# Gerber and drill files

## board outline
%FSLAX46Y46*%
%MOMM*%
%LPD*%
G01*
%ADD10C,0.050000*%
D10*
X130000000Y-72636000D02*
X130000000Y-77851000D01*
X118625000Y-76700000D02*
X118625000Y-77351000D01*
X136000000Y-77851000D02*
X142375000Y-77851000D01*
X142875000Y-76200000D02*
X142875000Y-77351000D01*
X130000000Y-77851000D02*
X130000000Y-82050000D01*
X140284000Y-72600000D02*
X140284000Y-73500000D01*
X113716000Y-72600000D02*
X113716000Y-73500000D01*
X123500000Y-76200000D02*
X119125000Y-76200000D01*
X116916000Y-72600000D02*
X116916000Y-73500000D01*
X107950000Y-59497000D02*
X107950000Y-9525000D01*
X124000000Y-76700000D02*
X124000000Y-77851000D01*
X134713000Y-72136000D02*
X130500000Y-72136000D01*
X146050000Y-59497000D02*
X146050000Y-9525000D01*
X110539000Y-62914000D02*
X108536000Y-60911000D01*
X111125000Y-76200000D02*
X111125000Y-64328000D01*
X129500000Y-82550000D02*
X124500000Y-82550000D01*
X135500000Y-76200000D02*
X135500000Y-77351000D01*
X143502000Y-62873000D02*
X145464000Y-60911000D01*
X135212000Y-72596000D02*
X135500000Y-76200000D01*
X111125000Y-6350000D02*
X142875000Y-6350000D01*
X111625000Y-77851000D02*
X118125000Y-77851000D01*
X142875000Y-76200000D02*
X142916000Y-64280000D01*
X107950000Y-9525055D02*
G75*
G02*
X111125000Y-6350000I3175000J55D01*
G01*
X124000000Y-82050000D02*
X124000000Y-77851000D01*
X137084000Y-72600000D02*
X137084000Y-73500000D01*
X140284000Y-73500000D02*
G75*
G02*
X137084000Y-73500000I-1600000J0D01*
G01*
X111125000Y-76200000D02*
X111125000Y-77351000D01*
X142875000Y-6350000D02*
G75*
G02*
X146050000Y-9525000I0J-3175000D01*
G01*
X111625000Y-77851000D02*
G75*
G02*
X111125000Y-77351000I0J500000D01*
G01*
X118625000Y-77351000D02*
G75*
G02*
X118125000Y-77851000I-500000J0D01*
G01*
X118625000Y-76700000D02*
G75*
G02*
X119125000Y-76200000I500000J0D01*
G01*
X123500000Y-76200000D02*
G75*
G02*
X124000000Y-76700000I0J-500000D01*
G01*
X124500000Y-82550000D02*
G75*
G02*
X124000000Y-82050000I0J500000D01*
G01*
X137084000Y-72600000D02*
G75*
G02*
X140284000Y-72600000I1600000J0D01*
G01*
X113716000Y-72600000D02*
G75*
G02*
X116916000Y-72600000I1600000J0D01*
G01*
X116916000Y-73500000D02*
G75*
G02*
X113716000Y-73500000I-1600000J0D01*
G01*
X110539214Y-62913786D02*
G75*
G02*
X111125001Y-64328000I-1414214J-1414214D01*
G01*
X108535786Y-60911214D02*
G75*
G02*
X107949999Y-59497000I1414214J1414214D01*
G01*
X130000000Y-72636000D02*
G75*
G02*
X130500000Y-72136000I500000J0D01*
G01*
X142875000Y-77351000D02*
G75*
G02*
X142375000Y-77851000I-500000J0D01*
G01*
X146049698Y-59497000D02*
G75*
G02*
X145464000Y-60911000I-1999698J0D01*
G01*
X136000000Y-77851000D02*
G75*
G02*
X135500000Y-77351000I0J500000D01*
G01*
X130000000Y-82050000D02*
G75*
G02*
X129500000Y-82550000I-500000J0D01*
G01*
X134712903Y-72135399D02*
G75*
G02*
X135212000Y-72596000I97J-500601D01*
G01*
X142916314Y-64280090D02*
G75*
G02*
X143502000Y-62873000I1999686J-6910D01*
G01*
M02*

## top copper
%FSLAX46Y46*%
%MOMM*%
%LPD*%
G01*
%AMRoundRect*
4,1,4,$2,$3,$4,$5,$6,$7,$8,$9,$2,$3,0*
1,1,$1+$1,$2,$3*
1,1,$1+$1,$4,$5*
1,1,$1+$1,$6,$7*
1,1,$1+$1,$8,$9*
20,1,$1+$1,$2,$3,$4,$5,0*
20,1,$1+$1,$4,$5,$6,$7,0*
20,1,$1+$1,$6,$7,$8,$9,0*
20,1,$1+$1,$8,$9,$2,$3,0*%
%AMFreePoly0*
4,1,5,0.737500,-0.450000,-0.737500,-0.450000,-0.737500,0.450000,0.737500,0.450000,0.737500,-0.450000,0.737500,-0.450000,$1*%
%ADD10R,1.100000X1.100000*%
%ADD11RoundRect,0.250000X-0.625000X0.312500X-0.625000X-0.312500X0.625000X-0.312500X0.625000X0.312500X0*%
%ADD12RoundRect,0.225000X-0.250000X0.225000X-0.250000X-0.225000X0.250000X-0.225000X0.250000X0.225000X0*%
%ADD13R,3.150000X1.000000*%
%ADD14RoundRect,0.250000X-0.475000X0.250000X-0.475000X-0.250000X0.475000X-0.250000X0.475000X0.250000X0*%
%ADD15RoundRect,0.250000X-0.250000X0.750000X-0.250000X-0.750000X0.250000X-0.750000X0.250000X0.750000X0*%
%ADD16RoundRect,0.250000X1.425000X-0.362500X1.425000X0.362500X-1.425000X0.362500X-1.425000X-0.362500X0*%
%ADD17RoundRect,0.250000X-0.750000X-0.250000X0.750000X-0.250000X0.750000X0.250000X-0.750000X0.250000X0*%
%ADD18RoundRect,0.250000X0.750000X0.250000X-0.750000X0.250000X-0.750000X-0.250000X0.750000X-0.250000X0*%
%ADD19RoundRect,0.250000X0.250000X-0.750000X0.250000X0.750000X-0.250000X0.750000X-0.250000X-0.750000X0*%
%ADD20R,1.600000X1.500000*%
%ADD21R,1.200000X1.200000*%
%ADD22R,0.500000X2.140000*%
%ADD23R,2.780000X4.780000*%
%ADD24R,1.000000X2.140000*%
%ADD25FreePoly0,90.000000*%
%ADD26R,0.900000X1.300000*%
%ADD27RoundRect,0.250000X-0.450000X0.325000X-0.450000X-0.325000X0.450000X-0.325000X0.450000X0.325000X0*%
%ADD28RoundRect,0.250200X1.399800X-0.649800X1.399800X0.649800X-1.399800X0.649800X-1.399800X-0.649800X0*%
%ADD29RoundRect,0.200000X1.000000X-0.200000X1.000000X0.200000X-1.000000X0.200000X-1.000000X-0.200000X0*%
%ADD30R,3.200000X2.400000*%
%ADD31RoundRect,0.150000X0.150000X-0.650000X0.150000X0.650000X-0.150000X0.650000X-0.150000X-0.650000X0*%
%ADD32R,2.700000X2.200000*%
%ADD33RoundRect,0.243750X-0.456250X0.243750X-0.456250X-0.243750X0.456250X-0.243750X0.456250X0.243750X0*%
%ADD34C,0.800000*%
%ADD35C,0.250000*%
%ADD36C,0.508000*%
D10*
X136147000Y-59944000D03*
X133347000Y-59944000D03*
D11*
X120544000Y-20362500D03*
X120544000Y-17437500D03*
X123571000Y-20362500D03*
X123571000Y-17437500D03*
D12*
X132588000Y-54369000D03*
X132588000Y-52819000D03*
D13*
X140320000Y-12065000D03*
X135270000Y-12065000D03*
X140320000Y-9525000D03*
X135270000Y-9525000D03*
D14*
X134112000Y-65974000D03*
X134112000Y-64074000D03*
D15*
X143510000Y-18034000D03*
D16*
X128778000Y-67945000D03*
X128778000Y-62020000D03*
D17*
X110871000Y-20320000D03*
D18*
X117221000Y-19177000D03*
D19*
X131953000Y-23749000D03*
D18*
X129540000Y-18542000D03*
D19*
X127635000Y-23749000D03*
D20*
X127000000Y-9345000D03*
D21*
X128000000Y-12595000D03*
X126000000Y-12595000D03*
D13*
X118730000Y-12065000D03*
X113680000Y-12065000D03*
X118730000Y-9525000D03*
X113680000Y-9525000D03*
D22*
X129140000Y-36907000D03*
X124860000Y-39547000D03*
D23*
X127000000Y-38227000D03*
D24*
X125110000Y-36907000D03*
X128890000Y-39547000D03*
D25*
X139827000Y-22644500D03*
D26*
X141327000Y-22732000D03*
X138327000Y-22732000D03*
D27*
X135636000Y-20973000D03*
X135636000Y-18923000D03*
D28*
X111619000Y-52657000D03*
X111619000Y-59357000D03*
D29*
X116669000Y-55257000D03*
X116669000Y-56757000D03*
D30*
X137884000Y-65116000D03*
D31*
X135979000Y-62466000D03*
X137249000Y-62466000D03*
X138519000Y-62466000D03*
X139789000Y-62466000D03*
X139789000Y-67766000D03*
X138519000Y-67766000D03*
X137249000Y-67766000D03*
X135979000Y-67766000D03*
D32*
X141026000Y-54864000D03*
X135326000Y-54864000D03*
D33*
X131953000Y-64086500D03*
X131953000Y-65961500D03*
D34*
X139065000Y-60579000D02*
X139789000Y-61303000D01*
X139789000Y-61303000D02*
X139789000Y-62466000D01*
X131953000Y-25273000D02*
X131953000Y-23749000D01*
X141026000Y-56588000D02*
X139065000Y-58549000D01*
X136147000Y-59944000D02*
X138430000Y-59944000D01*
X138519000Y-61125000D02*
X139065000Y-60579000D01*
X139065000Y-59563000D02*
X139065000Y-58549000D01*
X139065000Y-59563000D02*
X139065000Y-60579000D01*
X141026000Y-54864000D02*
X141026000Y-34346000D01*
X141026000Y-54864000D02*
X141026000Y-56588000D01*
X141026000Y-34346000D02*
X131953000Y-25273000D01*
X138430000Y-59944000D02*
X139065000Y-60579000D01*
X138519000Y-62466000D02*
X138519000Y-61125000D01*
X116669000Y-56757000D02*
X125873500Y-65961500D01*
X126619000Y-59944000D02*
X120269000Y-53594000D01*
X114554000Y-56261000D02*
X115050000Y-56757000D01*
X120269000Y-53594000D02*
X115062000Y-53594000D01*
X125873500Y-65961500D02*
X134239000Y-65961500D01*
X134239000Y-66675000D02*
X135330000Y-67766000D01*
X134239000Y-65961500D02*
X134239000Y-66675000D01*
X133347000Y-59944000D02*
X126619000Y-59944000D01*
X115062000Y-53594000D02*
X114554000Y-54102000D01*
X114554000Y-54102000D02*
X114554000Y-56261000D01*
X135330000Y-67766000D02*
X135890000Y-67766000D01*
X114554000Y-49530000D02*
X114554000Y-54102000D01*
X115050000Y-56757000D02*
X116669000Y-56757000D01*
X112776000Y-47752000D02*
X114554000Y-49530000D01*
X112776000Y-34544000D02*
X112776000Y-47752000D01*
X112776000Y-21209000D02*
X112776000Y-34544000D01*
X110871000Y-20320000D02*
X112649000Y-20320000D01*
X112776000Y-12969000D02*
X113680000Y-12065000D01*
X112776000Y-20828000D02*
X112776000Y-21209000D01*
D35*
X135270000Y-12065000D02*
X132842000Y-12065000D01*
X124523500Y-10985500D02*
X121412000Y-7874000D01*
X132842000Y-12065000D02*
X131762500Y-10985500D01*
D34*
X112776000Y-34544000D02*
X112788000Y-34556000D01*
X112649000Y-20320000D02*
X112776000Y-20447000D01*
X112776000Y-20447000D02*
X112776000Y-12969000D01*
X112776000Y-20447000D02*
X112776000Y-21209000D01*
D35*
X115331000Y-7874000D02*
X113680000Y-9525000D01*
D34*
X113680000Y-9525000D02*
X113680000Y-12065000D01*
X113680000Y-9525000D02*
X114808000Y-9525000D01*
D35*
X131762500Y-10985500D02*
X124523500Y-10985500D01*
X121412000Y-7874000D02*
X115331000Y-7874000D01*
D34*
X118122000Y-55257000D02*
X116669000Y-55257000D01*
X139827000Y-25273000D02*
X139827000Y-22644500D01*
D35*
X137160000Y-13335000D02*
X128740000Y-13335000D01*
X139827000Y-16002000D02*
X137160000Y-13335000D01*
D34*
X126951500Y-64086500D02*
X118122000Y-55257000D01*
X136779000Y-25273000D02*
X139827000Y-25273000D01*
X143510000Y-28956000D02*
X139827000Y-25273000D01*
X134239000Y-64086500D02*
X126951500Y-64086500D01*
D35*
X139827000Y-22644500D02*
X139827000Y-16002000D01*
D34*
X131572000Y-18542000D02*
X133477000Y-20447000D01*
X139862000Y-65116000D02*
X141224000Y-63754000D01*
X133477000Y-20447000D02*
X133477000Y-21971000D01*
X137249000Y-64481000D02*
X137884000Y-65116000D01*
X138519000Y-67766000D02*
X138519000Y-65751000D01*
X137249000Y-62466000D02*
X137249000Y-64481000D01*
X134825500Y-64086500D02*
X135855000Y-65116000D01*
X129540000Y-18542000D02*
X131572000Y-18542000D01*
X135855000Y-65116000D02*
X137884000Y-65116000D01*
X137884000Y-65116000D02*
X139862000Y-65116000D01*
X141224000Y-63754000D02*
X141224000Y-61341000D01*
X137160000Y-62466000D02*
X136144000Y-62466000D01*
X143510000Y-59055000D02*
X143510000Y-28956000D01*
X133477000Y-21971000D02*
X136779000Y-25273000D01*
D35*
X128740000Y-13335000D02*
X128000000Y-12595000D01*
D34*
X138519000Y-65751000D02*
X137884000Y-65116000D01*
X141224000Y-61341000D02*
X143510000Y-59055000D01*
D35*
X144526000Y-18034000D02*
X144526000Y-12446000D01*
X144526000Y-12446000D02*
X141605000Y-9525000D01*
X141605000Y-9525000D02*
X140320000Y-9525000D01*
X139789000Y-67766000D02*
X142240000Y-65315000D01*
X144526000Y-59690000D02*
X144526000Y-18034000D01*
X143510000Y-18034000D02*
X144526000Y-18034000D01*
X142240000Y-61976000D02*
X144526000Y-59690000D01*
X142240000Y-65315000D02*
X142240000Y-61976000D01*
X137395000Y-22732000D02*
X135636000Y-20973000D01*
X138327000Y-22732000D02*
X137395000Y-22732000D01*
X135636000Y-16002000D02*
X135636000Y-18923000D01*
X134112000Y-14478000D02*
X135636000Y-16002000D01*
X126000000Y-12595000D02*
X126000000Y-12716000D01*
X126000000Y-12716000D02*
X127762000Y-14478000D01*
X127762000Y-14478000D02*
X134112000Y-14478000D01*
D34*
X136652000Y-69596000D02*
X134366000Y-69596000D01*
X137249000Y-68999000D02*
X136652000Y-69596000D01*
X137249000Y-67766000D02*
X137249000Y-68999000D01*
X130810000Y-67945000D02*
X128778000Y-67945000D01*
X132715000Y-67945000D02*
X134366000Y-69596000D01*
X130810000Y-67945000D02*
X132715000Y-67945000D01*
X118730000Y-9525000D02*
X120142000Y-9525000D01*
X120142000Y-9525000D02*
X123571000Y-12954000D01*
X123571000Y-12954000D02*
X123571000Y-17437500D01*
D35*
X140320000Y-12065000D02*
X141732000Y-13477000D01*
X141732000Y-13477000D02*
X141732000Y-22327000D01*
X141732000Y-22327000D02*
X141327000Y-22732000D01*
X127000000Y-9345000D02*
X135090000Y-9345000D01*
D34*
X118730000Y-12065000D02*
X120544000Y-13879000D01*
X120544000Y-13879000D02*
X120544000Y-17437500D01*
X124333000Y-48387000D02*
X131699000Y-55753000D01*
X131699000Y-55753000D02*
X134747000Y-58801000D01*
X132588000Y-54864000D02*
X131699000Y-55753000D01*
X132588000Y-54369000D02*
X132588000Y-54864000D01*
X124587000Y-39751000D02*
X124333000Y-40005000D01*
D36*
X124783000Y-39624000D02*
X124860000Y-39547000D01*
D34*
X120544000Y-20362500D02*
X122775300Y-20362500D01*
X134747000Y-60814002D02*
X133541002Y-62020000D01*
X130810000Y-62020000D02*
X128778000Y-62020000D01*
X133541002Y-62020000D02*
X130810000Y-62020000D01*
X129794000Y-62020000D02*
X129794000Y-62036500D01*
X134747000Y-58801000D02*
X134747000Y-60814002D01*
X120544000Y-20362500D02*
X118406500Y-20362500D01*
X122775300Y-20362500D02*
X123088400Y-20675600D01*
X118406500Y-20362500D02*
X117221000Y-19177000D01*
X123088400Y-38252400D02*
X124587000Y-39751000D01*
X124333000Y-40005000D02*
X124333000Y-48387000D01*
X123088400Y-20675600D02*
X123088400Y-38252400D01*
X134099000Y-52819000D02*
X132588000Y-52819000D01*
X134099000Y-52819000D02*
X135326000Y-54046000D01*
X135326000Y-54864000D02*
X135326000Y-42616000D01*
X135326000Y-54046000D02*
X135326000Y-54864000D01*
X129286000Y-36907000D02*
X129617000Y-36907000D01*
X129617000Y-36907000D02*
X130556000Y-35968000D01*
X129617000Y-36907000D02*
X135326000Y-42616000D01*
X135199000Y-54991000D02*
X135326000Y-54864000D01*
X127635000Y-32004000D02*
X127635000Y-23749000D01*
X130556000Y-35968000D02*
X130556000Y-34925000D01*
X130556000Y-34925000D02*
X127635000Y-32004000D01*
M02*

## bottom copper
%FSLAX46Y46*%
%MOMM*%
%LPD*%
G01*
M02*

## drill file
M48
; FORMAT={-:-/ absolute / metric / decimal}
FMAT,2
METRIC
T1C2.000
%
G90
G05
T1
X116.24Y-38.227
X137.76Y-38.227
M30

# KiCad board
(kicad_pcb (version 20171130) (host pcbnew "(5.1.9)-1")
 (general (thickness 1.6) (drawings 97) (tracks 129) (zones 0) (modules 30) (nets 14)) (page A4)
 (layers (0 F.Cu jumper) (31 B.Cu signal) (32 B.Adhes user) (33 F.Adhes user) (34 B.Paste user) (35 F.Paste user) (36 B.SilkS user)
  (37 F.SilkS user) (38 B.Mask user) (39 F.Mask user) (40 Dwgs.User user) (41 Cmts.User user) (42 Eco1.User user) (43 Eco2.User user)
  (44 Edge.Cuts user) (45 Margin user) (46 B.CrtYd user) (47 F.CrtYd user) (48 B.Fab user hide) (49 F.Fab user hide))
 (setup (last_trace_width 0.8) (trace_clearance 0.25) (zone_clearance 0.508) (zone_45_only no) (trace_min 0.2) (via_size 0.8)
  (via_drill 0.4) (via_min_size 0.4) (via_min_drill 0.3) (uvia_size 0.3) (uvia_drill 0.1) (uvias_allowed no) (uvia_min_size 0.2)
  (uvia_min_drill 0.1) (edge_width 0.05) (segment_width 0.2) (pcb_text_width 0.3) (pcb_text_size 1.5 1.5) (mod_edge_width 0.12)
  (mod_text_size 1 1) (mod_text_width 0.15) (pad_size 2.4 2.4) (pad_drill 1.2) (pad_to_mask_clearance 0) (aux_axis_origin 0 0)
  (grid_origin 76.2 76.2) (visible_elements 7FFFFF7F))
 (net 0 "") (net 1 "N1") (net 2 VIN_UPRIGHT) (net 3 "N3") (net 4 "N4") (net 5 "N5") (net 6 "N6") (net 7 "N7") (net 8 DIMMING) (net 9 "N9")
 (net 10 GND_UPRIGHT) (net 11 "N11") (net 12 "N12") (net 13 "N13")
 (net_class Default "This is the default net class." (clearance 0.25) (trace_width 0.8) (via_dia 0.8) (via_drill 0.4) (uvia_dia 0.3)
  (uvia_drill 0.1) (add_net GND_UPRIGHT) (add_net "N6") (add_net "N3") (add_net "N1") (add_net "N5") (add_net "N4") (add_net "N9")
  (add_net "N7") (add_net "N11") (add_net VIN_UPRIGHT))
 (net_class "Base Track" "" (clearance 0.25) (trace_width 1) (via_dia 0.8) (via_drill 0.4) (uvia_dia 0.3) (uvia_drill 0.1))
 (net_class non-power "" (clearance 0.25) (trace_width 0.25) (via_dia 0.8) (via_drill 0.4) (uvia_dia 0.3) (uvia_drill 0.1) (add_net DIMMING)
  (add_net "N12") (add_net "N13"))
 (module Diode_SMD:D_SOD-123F (layer F.Cu) (at 134.747 59.944)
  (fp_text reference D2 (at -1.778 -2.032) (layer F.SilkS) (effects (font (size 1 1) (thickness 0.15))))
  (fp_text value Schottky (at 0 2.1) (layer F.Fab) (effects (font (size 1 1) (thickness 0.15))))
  (pad 2 smd rect (at 1.4 0) (size 1.1 1.1) (layers F.Cu F.Paste F.Mask) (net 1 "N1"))
  (pad 1 smd rect (at -1.4 0) (size 1.1 1.1) (layers F.Cu F.Paste F.Mask) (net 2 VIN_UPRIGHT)))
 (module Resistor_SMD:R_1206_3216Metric (layer F.Cu) (at 120.544 18.9 270)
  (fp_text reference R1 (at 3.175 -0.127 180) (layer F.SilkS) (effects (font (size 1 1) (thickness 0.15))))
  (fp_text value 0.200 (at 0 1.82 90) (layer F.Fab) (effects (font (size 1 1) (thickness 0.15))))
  (pad 2 smd roundrect (at 1.4625 0 270) (size 1.125 1.75) (layers F.Cu F.Paste F.Mask) (roundrect_rratio 0.222222) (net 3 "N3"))
  (pad 1 smd roundrect (at -1.4625 0 270) (size 1.125 1.75) (layers F.Cu F.Paste F.Mask) (roundrect_rratio 0.222222) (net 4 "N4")))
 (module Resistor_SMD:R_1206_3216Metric (layer F.Cu) (at 123.571 18.9 270)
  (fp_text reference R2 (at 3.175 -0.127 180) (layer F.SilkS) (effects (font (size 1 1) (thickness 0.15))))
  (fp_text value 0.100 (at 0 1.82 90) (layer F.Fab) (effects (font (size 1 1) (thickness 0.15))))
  (pad 2 smd roundrect (at 1.4625 0 270) (size 1.125 1.75) (layers F.Cu F.Paste F.Mask) (roundrect_rratio 0.222222) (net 3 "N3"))
  (pad 1 smd roundrect (at -1.4625 0 270) (size 1.125 1.75) (layers F.Cu F.Paste F.Mask) (roundrect_rratio 0.222222) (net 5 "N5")))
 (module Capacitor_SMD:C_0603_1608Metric (layer F.Cu) (at 132.588 53.594 270)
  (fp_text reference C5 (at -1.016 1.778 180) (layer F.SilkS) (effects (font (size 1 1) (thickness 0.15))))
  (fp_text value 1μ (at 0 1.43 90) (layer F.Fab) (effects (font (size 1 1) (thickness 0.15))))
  (pad 2 smd roundrect (at 0.775 0 270) (size 0.9 0.95) (layers F.Cu F.Paste F.Mask) (roundrect_rratio 0.25) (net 3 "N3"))
  (pad 1 smd roundrect (at -0.775 0 270) (size 0.9 0.95) (layers F.Cu F.Paste F.Mask) (roundrect_rratio 0.25) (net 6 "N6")))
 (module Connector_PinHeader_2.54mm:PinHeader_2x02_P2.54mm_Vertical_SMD (layer F.Cu) (at 137.795 10.795)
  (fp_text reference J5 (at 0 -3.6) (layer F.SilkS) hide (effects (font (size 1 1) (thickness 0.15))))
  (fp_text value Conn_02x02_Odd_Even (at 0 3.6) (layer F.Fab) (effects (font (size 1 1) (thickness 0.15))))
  (pad 4 smd rect (at 2.525 1.27) (size 3.15 1) (layers F.Cu F.Paste F.Mask) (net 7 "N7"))
  (pad 3 smd rect (at -2.525 1.27) (size 3.15 1) (layers F.Cu F.Paste F.Mask) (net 2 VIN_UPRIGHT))
  (pad 1 smd rect (at 2.525 -1.27) (size 3.15 1) (layers F.Cu F.Paste F.Mask) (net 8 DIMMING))
  (pad 2 smd rect (at -2.525 -1.27) (size 3.15 1) (layers F.Cu F.Paste F.Mask) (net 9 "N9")))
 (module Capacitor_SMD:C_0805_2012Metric (layer F.Cu) (at 134.112 65.024 270)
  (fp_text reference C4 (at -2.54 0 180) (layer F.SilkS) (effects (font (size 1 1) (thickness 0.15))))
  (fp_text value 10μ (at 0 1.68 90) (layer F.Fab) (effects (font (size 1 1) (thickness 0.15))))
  (pad 2 smd roundrect (at 0.95 0 270) (size 1 1.45) (layers F.Cu F.Paste F.Mask) (roundrect_rratio 0.25) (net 2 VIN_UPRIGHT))
  (pad 1 smd roundrect (at -0.95 0 270) (size 1 1.45) (layers F.Cu F.Paste F.Mask) (roundrect_rratio 0.25) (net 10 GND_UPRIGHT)))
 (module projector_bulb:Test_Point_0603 (layer F.Cu) (at 143.51 18.034 270)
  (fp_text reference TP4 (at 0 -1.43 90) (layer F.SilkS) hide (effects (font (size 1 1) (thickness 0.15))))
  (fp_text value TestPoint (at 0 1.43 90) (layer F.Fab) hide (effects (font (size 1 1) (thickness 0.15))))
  (pad 1 smd roundrect (at 0 0 270) (size 2 1) (layers F.Cu F.Paste F.Mask) (roundrect_rratio 0.25) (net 8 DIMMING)))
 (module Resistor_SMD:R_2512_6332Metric (layer F.Cu) (at 128.778 64.9825 90)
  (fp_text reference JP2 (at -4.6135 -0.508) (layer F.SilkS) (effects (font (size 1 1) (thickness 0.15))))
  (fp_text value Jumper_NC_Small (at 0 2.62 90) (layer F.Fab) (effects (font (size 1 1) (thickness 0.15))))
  (pad 1 smd roundrect (at -2.9625 0 90) (size 1.225 3.35) (layers F.Cu F.Paste F.Mask) (roundrect_rratio 0.204082) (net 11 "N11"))
  (pad 2 smd roundrect (at 2.9625 0 90) (size 1.225 3.35) (layers F.Cu F.Paste F.Mask) (roundrect_rratio 0.204082) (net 3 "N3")))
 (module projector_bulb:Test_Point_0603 (layer F.Cu) (at 110.871 20.32)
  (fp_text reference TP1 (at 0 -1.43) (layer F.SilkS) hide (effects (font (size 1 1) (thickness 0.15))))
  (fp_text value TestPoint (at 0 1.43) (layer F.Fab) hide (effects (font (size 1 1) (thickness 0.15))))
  (pad 1 smd roundrect (at 0 0) (size 2 1) (layers F.Cu F.Paste F.Mask) (roundrect_rratio 0.25) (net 2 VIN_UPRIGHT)))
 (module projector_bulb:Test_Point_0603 (layer F.Cu) (at 117.221 19.177 180)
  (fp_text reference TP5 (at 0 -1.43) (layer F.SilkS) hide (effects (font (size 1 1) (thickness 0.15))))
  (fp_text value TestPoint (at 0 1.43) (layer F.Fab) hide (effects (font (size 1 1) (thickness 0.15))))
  (pad 1 smd roundrect (at 0 0 180) (size 2 1) (layers F.Cu F.Paste F.Mask) (roundrect_rratio 0.25) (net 3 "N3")))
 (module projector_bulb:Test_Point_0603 (layer F.Cu) (at 131.953 23.749 90)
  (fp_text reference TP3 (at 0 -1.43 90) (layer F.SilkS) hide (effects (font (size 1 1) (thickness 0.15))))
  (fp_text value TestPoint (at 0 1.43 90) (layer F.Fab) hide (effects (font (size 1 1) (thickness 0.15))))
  (pad 1 smd roundrect (at 0 0 90) (size 2 1) (layers F.Cu F.Paste F.Mask) (roundrect_rratio 0.25) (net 1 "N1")))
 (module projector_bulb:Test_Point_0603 (layer F.Cu) (at 129.54 18.542 180)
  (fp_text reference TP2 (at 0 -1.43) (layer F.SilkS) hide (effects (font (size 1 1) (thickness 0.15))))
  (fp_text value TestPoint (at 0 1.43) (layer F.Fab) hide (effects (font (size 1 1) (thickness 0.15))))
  (pad 1 smd roundrect (at 0 0 180) (size 2 1) (layers F.Cu F.Paste F.Mask) (roundrect_rratio 0.25) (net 10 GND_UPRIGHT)))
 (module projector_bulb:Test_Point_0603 (layer F.Cu) (at 127.635 23.749 90)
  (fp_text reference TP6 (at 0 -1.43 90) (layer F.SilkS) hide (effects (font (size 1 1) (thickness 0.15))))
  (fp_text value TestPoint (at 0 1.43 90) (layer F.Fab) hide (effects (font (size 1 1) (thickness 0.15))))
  (pad 1 smd roundrect (at 0 0 90) (size 2 1) (layers F.Cu F.Paste F.Mask) (roundrect_rratio 0.25) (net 6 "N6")))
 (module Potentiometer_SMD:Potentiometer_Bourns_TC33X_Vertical (layer F.Cu) (at 127 10.795 90)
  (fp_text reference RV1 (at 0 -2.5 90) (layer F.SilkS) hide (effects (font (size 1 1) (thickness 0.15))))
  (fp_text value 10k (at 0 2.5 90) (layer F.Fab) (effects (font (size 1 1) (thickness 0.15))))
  (pad 2 smd rect (at 1.45 0 90) (size 1.5 1.6) (layers F.Cu F.Paste F.Mask) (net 9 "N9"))
  (pad 3 smd rect (at -1.8 1 90) (size 1.2 1.2) (layers F.Cu F.Paste F.Mask) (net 10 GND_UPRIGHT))
  (pad 1 smd rect (at -1.8 -1 90) (size 1.2 1.2) (layers F.Cu F.Paste F.Mask) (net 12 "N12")))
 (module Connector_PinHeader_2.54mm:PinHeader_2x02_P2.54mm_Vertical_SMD (layer F.Cu) (at 116.205 10.795)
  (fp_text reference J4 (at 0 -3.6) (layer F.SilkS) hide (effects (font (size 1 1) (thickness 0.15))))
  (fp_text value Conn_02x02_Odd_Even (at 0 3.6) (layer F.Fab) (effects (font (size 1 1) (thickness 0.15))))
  (pad 4 smd rect (at 2.525 1.27) (size 3.15 1) (layers F.Cu F.Paste F.Mask) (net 4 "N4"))
  (pad 3 smd rect (at -2.525 1.27) (size 3.15 1) (layers F.Cu F.Paste F.Mask) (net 2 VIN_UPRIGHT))
  (pad 2 smd rect (at 2.525 -1.27) (size 3.15 1) (layers F.Cu F.Paste F.Mask) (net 5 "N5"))
  (pad 1 smd rect (at -2.525 -1.27) (size 3.15 1) (layers F.Cu F.Paste F.Mask) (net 2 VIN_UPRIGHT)))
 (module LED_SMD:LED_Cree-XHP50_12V (layer F.Cu) (at 127 38.227 180)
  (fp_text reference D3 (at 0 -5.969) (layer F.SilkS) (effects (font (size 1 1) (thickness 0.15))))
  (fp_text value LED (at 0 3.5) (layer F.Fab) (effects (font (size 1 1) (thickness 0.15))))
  (pad 1 smd rect (at -2.14 1.32 180) (size 0.5 2.14) (layers F.Cu F.Paste F.Mask) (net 6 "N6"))
  (pad 2 smd rect (at 2.14 -1.32 180) (size 0.5 2.14) (layers F.Cu F.Paste F.Mask) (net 3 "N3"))
  (pad 3 smd rect (at 0 0 180) (size 2.78 4.78) (layers F.Cu F.Mask))
  (pad 3 smd rect (at 1.89 1.32 180) (size 1 2.14) (layers F.Cu F.Mask))
  (pad 3 smd rect (at -1.89 -1.32 180) (size 1 2.14) (layers F.Cu F.Mask))
  (pad "" smd rect (at -2.14 -1.32 180) (size 0.5 2.14) (layers F.Paste))
  (pad "" smd rect (at 2.14 1.32 180) (size 0.5 2.14) (layers F.Paste))
  (pad "" smd rect (at -0.61 -1.575 180) (size 0.97 0.8) (layers F.Paste))
  (pad "" smd rect (at 0.61 -1.575 180) (size 0.97 0.8) (layers F.Paste))
  (pad "" smd rect (at -0.61 -0.525 180) (size 0.97 0.8) (layers F.Paste))
  (pad "" smd rect (at 0.61 -0.525 180) (size 0.97 0.8) (layers F.Paste))
  (pad "" smd rect (at -0.61 0.525 180) (size 0.97 0.8) (layers F.Paste))
  (pad "" smd rect (at 0.61 0.525 180) (size 0.97 0.8) (layers F.Paste))
  (pad "" smd rect (at -0.61 1.575 180) (size 0.97 0.8) (layers F.Paste))
  (pad "" smd rect (at 0.61 1.575 180) (size 0.97 0.8) (layers F.Paste)))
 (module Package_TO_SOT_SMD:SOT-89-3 (layer F.Cu) (at 139.827 21.082 90)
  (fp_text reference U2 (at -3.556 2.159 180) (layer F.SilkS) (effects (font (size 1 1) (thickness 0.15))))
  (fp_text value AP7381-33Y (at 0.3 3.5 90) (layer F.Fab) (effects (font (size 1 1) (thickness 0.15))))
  (pad 2 smd custom (at -1.5625 0 90) (size 1.475 0.9) (layers F.Cu F.Paste F.Mask) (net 10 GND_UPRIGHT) (zone_connect 2)
   (options (clearance outline) (anchor rect)) (primitives))
  (pad 3 smd rect (at -1.65 1.5 90) (size 1.3 0.9) (layers F.Cu F.Paste F.Mask) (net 7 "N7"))
  (pad 1 smd rect (at -1.65 -1.5 90) (size 1.3 0.9) (layers F.Cu F.Paste F.Mask) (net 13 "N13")))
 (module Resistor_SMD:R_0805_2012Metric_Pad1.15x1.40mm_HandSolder (layer F.Cu) (at 135.636 19.948 270)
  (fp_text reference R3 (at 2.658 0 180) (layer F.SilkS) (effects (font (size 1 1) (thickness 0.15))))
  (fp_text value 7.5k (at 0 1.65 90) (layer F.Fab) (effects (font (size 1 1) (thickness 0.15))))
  (pad 2 smd roundrect (at 1.025 0 270) (size 1.15 1.4) (layers F.Cu F.Paste F.Mask) (roundrect_rratio 0.217391) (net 13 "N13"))
  (pad 1 smd roundrect (at -1.025 0 270) (size 1.15 1.4) (layers F.Cu F.Paste F.Mask) (roundrect_rratio 0.217391) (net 12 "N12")))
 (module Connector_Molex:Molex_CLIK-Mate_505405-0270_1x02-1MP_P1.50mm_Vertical (layer F.Cu) (at 113.919 56.007 90)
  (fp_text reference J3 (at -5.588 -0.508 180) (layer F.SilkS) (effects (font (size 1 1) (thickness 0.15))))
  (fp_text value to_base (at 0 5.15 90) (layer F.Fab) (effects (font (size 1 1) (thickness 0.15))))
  (pad "" smd roundrect (at 3.35 -2.3 90) (size 1.8 3.3) (layers F.Cu F.Paste F.Mask) (roundrect_rratio 0.139))
  (pad "" smd roundrect (at -3.35 -2.3 90) (size 1.8 3.3) (layers F.Cu F.Paste F.Mask) (roundrect_rratio 0.139))
  (pad 2 smd roundrect (at 0.75 2.75 90) (size 0.8 2.4) (layers F.Cu F.Paste F.Mask) (roundrect_rratio 0.25) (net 10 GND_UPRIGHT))
  (pad 1 smd roundrect (at -0.75 2.75 90) (size 0.8 2.4) (layers F.Cu F.Paste F.Mask) (roundrect_rratio 0.25) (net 2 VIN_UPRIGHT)))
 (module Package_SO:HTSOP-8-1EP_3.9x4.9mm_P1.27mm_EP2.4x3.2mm (layer F.Cu) (at 137.884 65.116 90)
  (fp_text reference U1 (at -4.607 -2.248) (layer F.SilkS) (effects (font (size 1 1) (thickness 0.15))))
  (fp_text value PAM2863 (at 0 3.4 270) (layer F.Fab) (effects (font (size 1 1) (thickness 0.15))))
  (pad "" smd roundrect (at 0.6 0.8 90) (size 0.97 1.29) (layers F.Paste) (roundrect_rratio 0.25))
  (pad "" smd roundrect (at 0.6 -0.8 90) (size 0.97 1.29) (layers F.Paste) (roundrect_rratio 0.25))
  (pad "" smd roundrect (at -0.6 0.8 90) (size 0.97 1.29) (layers F.Paste) (roundrect_rratio 0.25))
  (pad "" smd roundrect (at -0.6 -0.8 90) (size 0.97 1.29) (layers F.Paste) (roundrect_rratio 0.25))
  (pad 9 smd rect (at 0 0 90) (size 2.4 3.2) (layers F.Cu F.Mask) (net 10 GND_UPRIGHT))
  (pad 8 smd roundrect (at 2.65 -1.905 90) (size 1.6 0.6) (layers F.Cu F.Paste F.Mask) (roundrect_rratio 0.25) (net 10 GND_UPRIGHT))
  (pad 7 smd roundrect (at 2.65 -0.635 90) (size 1.6 0.6) (layers F.Cu F.Paste F.Mask) (roundrect_rratio 0.25) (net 10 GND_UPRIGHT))
  (pad 6 smd roundrect (at 2.65 0.635 90) (size 1.6 0.6) (layers F.Cu F.Paste F.Mask) (roundrect_rratio 0.25) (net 1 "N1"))
  (pad 5 smd roundrect (at 2.65 1.905 90) (size 1.6 0.6) (layers F.Cu F.Paste F.Mask) (roundrect_rratio 0.25) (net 1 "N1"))
  (pad 4 smd roundrect (at -2.65 1.905 90) (size 1.6 0.6) (layers F.Cu F.Paste F.Mask) (roundrect_rratio 0.25) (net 8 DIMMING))
  (pad 3 smd roundrect (at -2.65 0.635 90) (size 1.6 0.6) (layers F.Cu F.Paste F.Mask) (roundrect_rratio 0.25) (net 10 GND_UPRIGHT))
  (pad 2 smd roundrect (at -2.65 -0.635 90) (size 1.6 0.6) (layers F.Cu F.Paste F.Mask) (roundrect_rratio 0.25) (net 11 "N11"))
  (pad 1 smd roundrect (at -2.65 -1.905 90) (size 1.6 0.6) (layers F.Cu F.Paste F.Mask) (roundrect_rratio 0.25) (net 2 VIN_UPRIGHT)))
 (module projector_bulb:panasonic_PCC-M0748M (layer F.Cu) (at 138.176 54.864)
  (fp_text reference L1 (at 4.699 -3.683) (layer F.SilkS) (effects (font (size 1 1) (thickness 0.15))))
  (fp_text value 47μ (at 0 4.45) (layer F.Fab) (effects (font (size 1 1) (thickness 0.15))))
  (pad 2 smd rect (at 2.85 0) (size 2.7 2.2) (layers F.Cu F.Paste F.Mask) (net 1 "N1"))
  (pad 1 smd rect (at -2.85 0) (size 2.7 2.2) (layers F.Cu F.Paste F.Mask) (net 6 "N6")))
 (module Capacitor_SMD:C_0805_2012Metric (layer F.Cu) (at 131.953 65.024 270)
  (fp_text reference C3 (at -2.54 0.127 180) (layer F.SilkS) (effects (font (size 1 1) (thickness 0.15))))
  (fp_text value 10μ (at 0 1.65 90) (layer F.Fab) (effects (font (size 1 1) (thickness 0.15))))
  (pad 1 smd roundrect (at -0.9375 0 270) (size 0.975 1.4) (layers F.Cu F.Paste F.Mask) (roundrect_rratio 0.25) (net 10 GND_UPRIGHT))
  (pad 2 smd roundrect (at 0.9375 0 270) (size 0.975 1.4) (layers F.Cu F.Paste F.Mask) (roundrect_rratio 0.25) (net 2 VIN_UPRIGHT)))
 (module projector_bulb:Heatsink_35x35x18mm (layer B.Cu) (at 127 33.02) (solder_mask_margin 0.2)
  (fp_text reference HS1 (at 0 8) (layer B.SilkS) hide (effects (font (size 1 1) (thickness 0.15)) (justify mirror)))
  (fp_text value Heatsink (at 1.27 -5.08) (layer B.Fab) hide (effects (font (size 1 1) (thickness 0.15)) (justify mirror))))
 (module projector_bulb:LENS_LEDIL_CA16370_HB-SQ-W (layer F.Cu) (at 127 38.227)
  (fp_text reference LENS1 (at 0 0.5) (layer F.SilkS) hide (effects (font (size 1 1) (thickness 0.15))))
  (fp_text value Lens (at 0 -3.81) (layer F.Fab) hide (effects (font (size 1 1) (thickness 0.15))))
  (pad "" np_thru_hole circle (at -10.76 0) (size 2 2) (drill 2) (layers *.Cu *.Mask))
  (pad "" np_thru_hole circle (at 10.76 0) (size 2 2) (drill 2) (layers *.Cu *.Mask)))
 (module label (layer F.Cu) (at 134.239 24.257)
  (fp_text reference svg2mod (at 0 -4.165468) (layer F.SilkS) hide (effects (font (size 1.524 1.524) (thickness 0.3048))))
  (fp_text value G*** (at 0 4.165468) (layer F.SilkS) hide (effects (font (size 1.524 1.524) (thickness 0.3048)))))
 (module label (layer F.Cu) (at 116.84 21.336)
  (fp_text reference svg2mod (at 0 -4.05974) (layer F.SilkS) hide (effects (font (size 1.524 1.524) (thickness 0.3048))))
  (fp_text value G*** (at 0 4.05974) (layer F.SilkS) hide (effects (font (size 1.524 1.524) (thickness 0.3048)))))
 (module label (layer F.Cu) (at 110.871 22.479)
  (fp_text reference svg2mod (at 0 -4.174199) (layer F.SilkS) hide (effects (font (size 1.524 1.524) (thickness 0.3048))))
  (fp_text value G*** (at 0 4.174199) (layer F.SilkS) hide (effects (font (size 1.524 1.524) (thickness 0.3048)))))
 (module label (layer F.Cu) (at 129.667 20.447)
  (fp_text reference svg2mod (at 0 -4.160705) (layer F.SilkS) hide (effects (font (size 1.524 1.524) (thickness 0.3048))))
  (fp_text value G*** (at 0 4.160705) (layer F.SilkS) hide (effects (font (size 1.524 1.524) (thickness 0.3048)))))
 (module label (layer F.Cu) (at 144.526 21.336 90)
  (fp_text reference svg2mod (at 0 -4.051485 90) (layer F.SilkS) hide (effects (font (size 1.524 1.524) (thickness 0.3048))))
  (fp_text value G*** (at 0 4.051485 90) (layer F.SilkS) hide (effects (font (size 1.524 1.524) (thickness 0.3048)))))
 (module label (layer F.Cu) (at 123.698 24.257)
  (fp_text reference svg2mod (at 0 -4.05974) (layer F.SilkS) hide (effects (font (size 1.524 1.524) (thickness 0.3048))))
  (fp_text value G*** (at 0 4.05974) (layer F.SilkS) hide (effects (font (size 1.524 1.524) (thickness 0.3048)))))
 (gr_line (start 130 72.636) (end 130 77.851) (angle 90) (layer Edge.Cuts) (width 0.05))
 (gr_line (start 118.625 76.7) (end 118.625 77.351) (angle 90) (layer Edge.Cuts) (width 0.05))
 (gr_line (start 136 77.851) (end 142.375 77.851) (angle 90) (layer Edge.Cuts) (width 0.05))
 (gr_line (start 142.875 76.2) (end 142.875 77.351) (angle 90) (layer Edge.Cuts) (width 0.05))
 (gr_line (start 130 77.851) (end 130 82.05) (angle 90) (layer Edge.Cuts) (width 0.05))
 (gr_line (start 140.284 72.6) (end 140.284 73.5) (angle 90) (layer Edge.Cuts) (width 0.05))
 (gr_line (start 113.716 72.6) (end 113.716 73.5) (angle 90) (layer Edge.Cuts) (width 0.05))
 (gr_line (start 123.5 76.2) (end 119.125 76.2) (angle 90) (layer Edge.Cuts) (width 0.05))
 (gr_line (start 116.916 72.6) (end 116.916 73.5) (angle 90) (layer Edge.Cuts) (width 0.05))
 (gr_line (start 107.95 59.497) (end 107.95 9.525) (angle 90) (layer Edge.Cuts) (width 0.05))
 (gr_line (start 124 76.7) (end 124 77.851) (angle 90) (layer Edge.Cuts) (width 0.05))
 (gr_line (start 134.713 72.136) (end 130.5 72.136) (angle 90) (layer Edge.Cuts) (width 0.05))
 (gr_line (start 146.05 59.497) (end 146.05 9.525) (angle 90) (layer Edge.Cuts) (width 0.05))
 (gr_line (start 110.539 62.914) (end 108.536 60.911) (angle 90) (layer Edge.Cuts) (width 0.05))
 (gr_line (start 111.125 76.2) (end 111.125 64.328) (angle 90) (layer Edge.Cuts) (width 0.05))
 (gr_line (start 129.5 82.55) (end 124.5 82.55) (angle 90) (layer Edge.Cuts) (width 0.05))
 (gr_line (start 135.5 76.2) (end 135.5 77.351) (angle 90) (layer Edge.Cuts) (width 0.05))
 (gr_line (start 143.502 62.873) (end 145.464 60.911) (angle 90) (layer Edge.Cuts) (width 0.05))
 (gr_line (start 135.212 72.596) (end 135.5 76.2) (angle 90) (layer Edge.Cuts) (width 0.05))
 (gr_line (start 111.125 6.35) (end 142.875 6.35) (angle 90) (layer Edge.Cuts) (width 0.05))
 (gr_line (start 111.625 77.851) (end 118.125 77.851) (angle 90) (layer Edge.Cuts) (width 0.05))
 (gr_line (start 142.875 76.2) (end 142.916 64.28) (angle 90) (layer Edge.Cuts) (width 0.05))
 (gr_arc (start 111.125 9.525) (end 111.125 6.35) (angle -90.001) (layer Edge.Cuts) (width 0.05))
 (gr_line (start 124 82.05) (end 124 77.851) (angle 90) (layer Edge.Cuts) (width 0.05))
 (gr_line (start 137.084 72.6) (end 137.084 73.5) (angle 90) (layer Edge.Cuts) (width 0.05))
 (gr_arc (start 138.684 73.5) (end 137.084 73.5) (angle -180) (layer Edge.Cuts) (width 0.05))
 (gr_line (start 111.125 76.2) (end 111.125 77.351) (angle 90) (layer Edge.Cuts) (width 0.05))
 (gr_arc (start 142.875 9.525) (end 146.05 9.525) (angle -90) (layer Edge.Cuts) (width 0.05))
 (gr_arc (start 111.625 77.351) (end 111.125 77.351) (angle -90) (layer Edge.Cuts) (width 0.05))
 (gr_arc (start 118.125 77.351) (end 118.125 77.851) (angle -90) (layer Edge.Cuts) (width 0.05))
 (gr_arc (start 119.125 76.7) (end 119.125 76.2) (angle -90) (layer Edge.Cuts) (width 0.05))
 (gr_arc (start 123.5 76.7) (end 124 76.7) (angle -90) (layer Edge.Cuts) (width 0.05))
 (gr_arc (start 124.5 82.05) (end 124 82.05) (angle -90) (layer Edge.Cuts) (width 0.05))
 (gr_arc (start 138.684 72.6) (end 140.284 72.6) (angle -180) (layer Edge.Cuts) (width 0.05))
 (gr_arc (start 115.316 72.6) (end 116.916 72.6) (angle -180) (layer Edge.Cuts) (width 0.05))
 (gr_arc (start 115.316 73.5) (end 113.716 73.5) (angle -180) (layer Edge.Cuts) (width 0.05))
 (gr_arc (start 109.125 64.328) (end 111.125 64.328) (angle -45) (layer Edge.Cuts) (width 0.05))
 (gr_arc (start 109.95 59.497) (end 107.95 59.497) (angle -45) (layer Edge.Cuts) (width 0.05))
 (gr_arc (start 130.5 72.636) (end 130.5 72.136) (angle -90) (layer Edge.Cuts) (width 0.05))
 (gr_arc (start 142.375 77.351) (end 142.375 77.851) (angle -90) (layer Edge.Cuts) (width 0.05))
 (gr_arc (start 144.05 59.497) (end 145.464 60.911) (angle -45) (layer Edge.Cuts) (width 0.05))
 (gr_arc (start 136 77.351) (end 135.5 77.351) (angle -90) (layer Edge.Cuts) (width 0.05))
 (gr_arc (start 129.5 82.05) (end 129.5 82.55) (angle -90) (layer Edge.Cuts) (width 0.05))
 (gr_arc (start 134.713 72.636) (end 135.212 72.596) (angle -85.428) (layer Edge.Cuts) (width 0.05))
 (gr_arc (start 144.916 64.287) (end 143.502 62.873) (angle -44.802) (layer Edge.Cuts) (width 0.05))
 (segment (start 139.065 60.579) (end 139.789 61.303) (width 0.8) (layer F.Cu) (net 1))
 (segment (start 139.789 61.303) (end 139.789 62.466) (width 0.8) (layer F.Cu) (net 1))
 (segment (start 131.953 25.273) (end 131.953 23.749) (width 0.8) (layer F.Cu) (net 1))
 (segment (start 141.026 56.588) (end 139.065 58.549) (width 0.8) (layer F.Cu) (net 1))
 (segment (start 136.147 59.944) (end 138.43 59.944) (width 0.8) (layer F.Cu) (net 1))
 (segment (start 138.519 61.125) (end 139.065 60.579) (width 0.8) (layer F.Cu) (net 1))
 (segment (start 139.065 59.563) (end 139.065 58.549) (width 0.8) (layer F.Cu) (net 1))
 (segment (start 139.065 59.563) (end 139.065 60.579) (width 0.8) (layer F.Cu) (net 1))
 (segment (start 141.026 54.864) (end 141.026 34.346) (width 0.8) (layer F.Cu) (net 1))
 (segment (start 141.026 54.864) (end 141.026 56.588) (width 0.8) (layer F.Cu) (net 1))
 (segment (start 141.026 34.346) (end 131.953 25.273) (width 0.8) (layer F.Cu) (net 1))
 (segment (start 138.43 59.944) (end 139.065 60.579) (width 0.8) (layer F.Cu) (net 1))
 (segment (start 138.519 62.466) (end 138.519 61.125) (width 0.8) (layer F.Cu) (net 1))
 (segment (start 116.669 56.757) (end 125.8735 65.9615) (width 0.8) (layer F.Cu) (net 2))
 (segment (start 126.619 59.944) (end 120.269 53.594) (width 0.8) (layer F.Cu) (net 2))
 (segment (start 114.554 56.261) (end 115.05 56.757) (width 0.8) (layer F.Cu) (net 2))
 (segment (start 120.269 53.594) (end 115.062 53.594) (width 0.8) (layer F.Cu) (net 2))
 (segment (start 125.8735 65.9615) (end 134.239 65.9615) (width 0.8) (layer F.Cu) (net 2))
 (segment (start 134.239 66.675) (end 135.33 67.766) (width 0.8) (layer F.Cu) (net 2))
 (segment (start 134.239 65.9615) (end 134.239 66.675) (width 0.8) (layer F.Cu) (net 2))
 (segment (start 133.347 59.944) (end 126.619 59.944) (width 0.8) (layer F.Cu) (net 2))
 (segment (start 115.062 53.594) (end 114.554 54.102) (width 0.8) (layer F.Cu) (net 2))
 (segment (start 114.554 54.102) (end 114.554 56.261) (width 0.8) (layer F.Cu) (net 2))
 (segment (start 135.33 67.766) (end 135.89 67.766) (width 0.8) (layer F.Cu) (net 2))
 (segment (start 114.554 49.53) (end 114.554 54.102) (width 0.8) (layer F.Cu) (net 2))
 (segment (start 115.05 56.757) (end 116.669 56.757) (width 0.8) (layer F.Cu) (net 2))
 (segment (start 112.776 47.752) (end 114.554 49.53) (width 0.8) (layer F.Cu) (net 2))
 (segment (start 112.776 34.544) (end 112.776 47.752) (width 0.8) (layer F.Cu) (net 2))
 (segment (start 112.776 21.209) (end 112.776 34.544) (width 0.8) (layer F.Cu) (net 2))
 (segment (start 110.871 20.32) (end 112.649 20.32) (width 0.8) (layer F.Cu) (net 2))
 (segment (start 112.776 12.969) (end 113.68 12.065) (width 0.8) (layer F.Cu) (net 2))
 (segment (start 112.776 20.828) (end 112.776 21.209) (width 0.8) (layer F.Cu) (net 2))
 (segment (start 135.27 12.065) (end 132.842 12.065) (width 0.25) (layer F.Cu) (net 2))
 (segment (start 124.5235 10.9855) (end 121.412 7.874) (width 0.25) (layer F.Cu) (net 2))
 (segment (start 132.842 12.065) (end 131.7625 10.9855) (width 0.25) (layer F.Cu) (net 2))
 (segment (start 112.776 34.544) (end 112.788 34.556) (width 0.8) (layer F.Cu) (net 2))
 (segment (start 112.649 20.32) (end 112.776 20.447) (width 0.8) (layer F.Cu) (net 2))
 (segment (start 112.776 20.447) (end 112.776 12.969) (width 0.8) (layer F.Cu) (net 2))
 (segment (start 112.776 20.447) (end 112.776 21.209) (width 0.8) (layer F.Cu) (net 2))
 (segment (start 115.331 7.874) (end 113.68 9.525) (width 0.25) (layer F.Cu) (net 2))
 (segment (start 113.68 9.525) (end 113.68 12.065) (width 0.8) (layer F.Cu) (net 2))
 (segment (start 113.68 9.525) (end 114.808 9.525) (width 0.8) (layer F.Cu) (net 2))
 (segment (start 131.7625 10.9855) (end 124.5235 10.9855) (width 0.25) (layer F.Cu) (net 2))
 (segment (start 121.412 7.874) (end 115.331 7.874) (width 0.25) (layer F.Cu) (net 2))
 (segment (start 118.122 55.257) (end 116.669 55.257) (width 0.8) (layer F.Cu) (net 10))
 (segment (start 139.827 25.273) (end 139.827 22.6445) (width 0.8) (layer F.Cu) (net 10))
 (segment (start 137.16 13.335) (end 128.74 13.335) (width 0.25) (layer F.Cu) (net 10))
 (segment (start 139.827 16.002) (end 137.16 13.335) (width 0.25) (layer F.Cu) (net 10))
 (segment (start 126.9515 64.0865) (end 118.122 55.257) (width 0.8) (layer F.Cu) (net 10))
 (segment (start 136.779 25.273) (end 139.827 25.273) (width 0.8) (layer F.Cu) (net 10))
 (segment (start 143.51 28.956) (end 139.827 25.273) (width 0.8) (layer F.Cu) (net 10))
 (segment (start 134.239 64.0865) (end 126.9515 64.0865) (width 0.8) (layer F.Cu) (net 10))
 (segment (start 139.827 22.6445) (end 139.827 16.002) (width 0.25) (layer F.Cu) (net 10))
 (segment (start 131.572 18.542) (end 133.477 20.447) (width 0.8) (layer F.Cu) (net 10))
 (segment (start 139.862 65.116) (end 141.224 63.754) (width 0.8) (layer F.Cu) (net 10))
 (segment (start 133.477 20.447) (end 133.477 21.971) (width 0.8) (layer F.Cu) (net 10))
 (segment (start 137.249 64.481) (end 137.884 65.116) (width 0.8) (layer F.Cu) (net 10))
 (segment (start 138.519 67.766) (end 138.519 65.751) (width 0.8) (layer F.Cu) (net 10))
 (segment (start 137.249 62.466) (end 137.249 64.481) (width 0.8) (layer F.Cu) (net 10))
 (segment (start 134.8255 64.0865) (end 135.855 65.116) (width 0.8) (layer F.Cu) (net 10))
 (segment (start 129.54 18.542) (end 131.572 18.542) (width 0.8) (layer F.Cu) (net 10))
 (segment (start 135.855 65.116) (end 137.884 65.116) (width 0.8) (layer F.Cu) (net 10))
 (segment (start 137.884 65.116) (end 139.862 65.116) (width 0.8) (layer F.Cu) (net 10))
 (segment (start 141.224 63.754) (end 141.224 61.341) (width 0.8) (layer F.Cu) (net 10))
 (segment (start 137.16 62.466) (end 136.144 62.466) (width 0.8) (layer F.Cu) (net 10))
 (segment (start 143.51 59.055) (end 143.51 28.956) (width 0.8) (layer F.Cu) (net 10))
 (segment (start 133.477 21.971) (end 136.779 25.273) (width 0.8) (layer F.Cu) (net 10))
 (segment (start 128.74 13.335) (end 128 12.595) (width 0.25) (layer F.Cu) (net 10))
 (segment (start 138.519 65.751) (end 137.884 65.116) (width 0.8) (layer F.Cu) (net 10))
 (segment (start 141.224 61.341) (end 143.51 59.055) (width 0.8) (layer F.Cu) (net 10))
 (segment (start 144.526 18.034) (end 144.526 12.446) (width 0.25) (layer F.Cu) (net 8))
 (segment (start 144.526 12.446) (end 141.605 9.525) (width 0.25) (layer F.Cu) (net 8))
 (segment (start 141.605 9.525) (end 140.32 9.525) (width 0.25) (layer F.Cu) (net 8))
 (segment (start 139.789 67.766) (end 142.24 65.315) (width 0.25) (layer F.Cu) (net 8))
 (segment (start 144.526 59.69) (end 144.526 18.034) (width 0.25) (layer F.Cu) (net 8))
 (segment (start 143.51 18.034) (end 144.526 18.034) (width 0.25) (layer F.Cu) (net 8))
 (segment (start 142.24 61.976) (end 144.526 59.69) (width 0.25) (layer F.Cu) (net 8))
 (segment (start 142.24 65.315) (end 142.24 61.976) (width 0.25) (layer F.Cu) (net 8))
 (segment (start 137.395 22.732) (end 135.636 20.973) (width 0.25) (layer F.Cu) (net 13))
 (segment (start 138.327 22.732) (end 137.395 22.732) (width 0.25) (layer F.Cu) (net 13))
 (segment (start 135.636 16.002) (end 135.636 18.923) (width 0.25) (layer F.Cu) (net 12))
 (segment (start 134.112 14.478) (end 135.636 16.002) (width 0.25) (layer F.Cu) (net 12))
 (segment (start 126 12.595) (end 126 12.716) (width 0.25) (layer F.Cu) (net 12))
 (segment (start 126 12.716) (end 127.762 14.478) (width 0.25) (layer F.Cu) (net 12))
 (segment (start 127.762 14.478) (end 134.112 14.478) (width 0.25) (layer F.Cu) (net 12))
 (segment (start 136.652 69.596) (end 134.366 69.596) (width 0.8) (layer F.Cu) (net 11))
 (segment (start 137.249 68.999) (end 136.652 69.596) (width 0.8) (layer F.Cu) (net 11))
 (segment (start 137.249 67.766) (end 137.249 68.999) (width 0.8) (layer F.Cu) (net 11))
 (segment (start 130.81 67.945) (end 128.778 67.945) (width 0.8) (layer F.Cu) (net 11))
 (segment (start 132.715 67.945) (end 134.366 69.596) (width 0.8) (layer F.Cu) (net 11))
 (segment (start 130.81 67.945) (end 132.715 67.945) (width 0.8) (layer F.Cu) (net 11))
 (segment (start 118.73 9.525) (end 120.142 9.525) (width 0.8) (layer F.Cu) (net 5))
 (segment (start 120.142 9.525) (end 123.571 12.954) (width 0.8) (layer F.Cu) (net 5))
 (segment (start 123.571 12.954) (end 123.571 17.4375) (width 0.8) (layer F.Cu) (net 5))
 (segment (start 140.32 12.065) (end 141.732 13.477) (width 0.25) (layer F.Cu) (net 7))
 (segment (start 141.732 13.477) (end 141.732 22.327) (width 0.25) (layer F.Cu) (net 7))
 (segment (start 141.732 22.327) (end 141.327 22.732) (width 0.25) (layer F.Cu) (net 7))
 (segment (start 127 9.345) (end 135.09 9.345) (width 0.25) (layer F.Cu) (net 9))
 (segment (start 118.73 12.065) (end 120.544 13.879) (width 0.8) (layer F.Cu) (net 4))
 (segment (start 120.544 13.879) (end 120.544 17.4375) (width 0.8) (layer F.Cu) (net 4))
 (segment (start 124.333 48.387) (end 131.699 55.753) (width 0.8) (layer F.Cu) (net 3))
 (segment (start 131.699 55.753) (end 134.747 58.801) (width 0.8) (layer F.Cu) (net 3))
 (segment (start 132.588 54.864) (end 131.699 55.753) (width 0.8) (layer F.Cu) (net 3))
 (segment (start 132.588 54.369) (end 132.588 54.864) (width 0.8) (layer F.Cu) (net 3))
 (segment (start 124.587 39.751) (end 124.333 40.005) (width 0.8) (layer F.Cu) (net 3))
 (segment (start 124.783 39.624) (end 124.86 39.547) (width 0.508) (layer F.Cu) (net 3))
 (segment (start 120.544 20.3625) (end 122.7753 20.3625) (width 0.8) (layer F.Cu) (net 3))
 (segment (start 134.747 60.814002) (end 133.541002 62.02) (width 0.8) (layer F.Cu) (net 3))
 (segment (start 130.81 62.02) (end 128.778 62.02) (width 0.8) (layer F.Cu) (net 3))
 (segment (start 133.541002 62.02) (end 130.81 62.02) (width 0.8) (layer F.Cu) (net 3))
 (segment (start 129.794 62.02) (end 129.794 62.0365) (width 0.8) (layer F.Cu) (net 3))
 (segment (start 134.747 58.801) (end 134.747 60.814002) (width 0.8) (layer F.Cu) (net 3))
 (segment (start 120.544 20.3625) (end 118.4065 20.3625) (width 0.8) (layer F.Cu) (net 3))
 (segment (start 122.7753 20.3625) (end 123.0884 20.6756) (width 0.8) (layer F.Cu) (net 3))
 (segment (start 118.4065 20.3625) (end 117.221 19.177) (width 0.8) (layer F.Cu) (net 3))
 (segment (start 123.0884 38.2524) (end 124.587 39.751) (width 0.8) (layer F.Cu) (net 3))
 (segment (start 124.333 40.005) (end 124.333 48.387) (width 0.8) (layer F.Cu) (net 3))
 (segment (start 123.0884 20.6756) (end 123.0884 38.2524) (width 0.8) (layer F.Cu) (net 3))
 (segment (start 134.099 52.819) (end 132.588 52.819) (width 0.8) (layer F.Cu) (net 6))
 (segment (start 134.099 52.819) (end 135.326 54.046) (width 0.8) (layer F.Cu) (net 6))
 (segment (start 135.326 54.864) (end 135.326 42.616) (width 0.8) (layer F.Cu) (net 6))
 (segment (start 135.326 54.046) (end 135.326 54.864) (width 0.8) (layer F.Cu) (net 6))
 (segment (start 129.286 36.907) (end 129.617 36.907) (width 0.8) (layer F.Cu) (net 6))
 (segment (start 129.617 36.907) (end 130.556 35.968) (width 0.8) (layer F.Cu) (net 6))
 (segment (start 129.617 36.907) (end 135.326 42.616) (width 0.8) (layer F.Cu) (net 6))
 (segment (start 135.199 54.991) (end 135.326 54.864) (width 0.8) (layer F.Cu) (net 6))
 (segment (start 127.635 32.004) (end 127.635 23.749) (width 0.8) (layer F.Cu) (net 6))
 (segment (start 130.556 35.968) (end 130.556 34.925) (width 0.8) (layer F.Cu) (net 6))
 (segment (start 130.556 34.925) (end 127.635 32.004) (width 0.8) (layer F.Cu) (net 6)))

